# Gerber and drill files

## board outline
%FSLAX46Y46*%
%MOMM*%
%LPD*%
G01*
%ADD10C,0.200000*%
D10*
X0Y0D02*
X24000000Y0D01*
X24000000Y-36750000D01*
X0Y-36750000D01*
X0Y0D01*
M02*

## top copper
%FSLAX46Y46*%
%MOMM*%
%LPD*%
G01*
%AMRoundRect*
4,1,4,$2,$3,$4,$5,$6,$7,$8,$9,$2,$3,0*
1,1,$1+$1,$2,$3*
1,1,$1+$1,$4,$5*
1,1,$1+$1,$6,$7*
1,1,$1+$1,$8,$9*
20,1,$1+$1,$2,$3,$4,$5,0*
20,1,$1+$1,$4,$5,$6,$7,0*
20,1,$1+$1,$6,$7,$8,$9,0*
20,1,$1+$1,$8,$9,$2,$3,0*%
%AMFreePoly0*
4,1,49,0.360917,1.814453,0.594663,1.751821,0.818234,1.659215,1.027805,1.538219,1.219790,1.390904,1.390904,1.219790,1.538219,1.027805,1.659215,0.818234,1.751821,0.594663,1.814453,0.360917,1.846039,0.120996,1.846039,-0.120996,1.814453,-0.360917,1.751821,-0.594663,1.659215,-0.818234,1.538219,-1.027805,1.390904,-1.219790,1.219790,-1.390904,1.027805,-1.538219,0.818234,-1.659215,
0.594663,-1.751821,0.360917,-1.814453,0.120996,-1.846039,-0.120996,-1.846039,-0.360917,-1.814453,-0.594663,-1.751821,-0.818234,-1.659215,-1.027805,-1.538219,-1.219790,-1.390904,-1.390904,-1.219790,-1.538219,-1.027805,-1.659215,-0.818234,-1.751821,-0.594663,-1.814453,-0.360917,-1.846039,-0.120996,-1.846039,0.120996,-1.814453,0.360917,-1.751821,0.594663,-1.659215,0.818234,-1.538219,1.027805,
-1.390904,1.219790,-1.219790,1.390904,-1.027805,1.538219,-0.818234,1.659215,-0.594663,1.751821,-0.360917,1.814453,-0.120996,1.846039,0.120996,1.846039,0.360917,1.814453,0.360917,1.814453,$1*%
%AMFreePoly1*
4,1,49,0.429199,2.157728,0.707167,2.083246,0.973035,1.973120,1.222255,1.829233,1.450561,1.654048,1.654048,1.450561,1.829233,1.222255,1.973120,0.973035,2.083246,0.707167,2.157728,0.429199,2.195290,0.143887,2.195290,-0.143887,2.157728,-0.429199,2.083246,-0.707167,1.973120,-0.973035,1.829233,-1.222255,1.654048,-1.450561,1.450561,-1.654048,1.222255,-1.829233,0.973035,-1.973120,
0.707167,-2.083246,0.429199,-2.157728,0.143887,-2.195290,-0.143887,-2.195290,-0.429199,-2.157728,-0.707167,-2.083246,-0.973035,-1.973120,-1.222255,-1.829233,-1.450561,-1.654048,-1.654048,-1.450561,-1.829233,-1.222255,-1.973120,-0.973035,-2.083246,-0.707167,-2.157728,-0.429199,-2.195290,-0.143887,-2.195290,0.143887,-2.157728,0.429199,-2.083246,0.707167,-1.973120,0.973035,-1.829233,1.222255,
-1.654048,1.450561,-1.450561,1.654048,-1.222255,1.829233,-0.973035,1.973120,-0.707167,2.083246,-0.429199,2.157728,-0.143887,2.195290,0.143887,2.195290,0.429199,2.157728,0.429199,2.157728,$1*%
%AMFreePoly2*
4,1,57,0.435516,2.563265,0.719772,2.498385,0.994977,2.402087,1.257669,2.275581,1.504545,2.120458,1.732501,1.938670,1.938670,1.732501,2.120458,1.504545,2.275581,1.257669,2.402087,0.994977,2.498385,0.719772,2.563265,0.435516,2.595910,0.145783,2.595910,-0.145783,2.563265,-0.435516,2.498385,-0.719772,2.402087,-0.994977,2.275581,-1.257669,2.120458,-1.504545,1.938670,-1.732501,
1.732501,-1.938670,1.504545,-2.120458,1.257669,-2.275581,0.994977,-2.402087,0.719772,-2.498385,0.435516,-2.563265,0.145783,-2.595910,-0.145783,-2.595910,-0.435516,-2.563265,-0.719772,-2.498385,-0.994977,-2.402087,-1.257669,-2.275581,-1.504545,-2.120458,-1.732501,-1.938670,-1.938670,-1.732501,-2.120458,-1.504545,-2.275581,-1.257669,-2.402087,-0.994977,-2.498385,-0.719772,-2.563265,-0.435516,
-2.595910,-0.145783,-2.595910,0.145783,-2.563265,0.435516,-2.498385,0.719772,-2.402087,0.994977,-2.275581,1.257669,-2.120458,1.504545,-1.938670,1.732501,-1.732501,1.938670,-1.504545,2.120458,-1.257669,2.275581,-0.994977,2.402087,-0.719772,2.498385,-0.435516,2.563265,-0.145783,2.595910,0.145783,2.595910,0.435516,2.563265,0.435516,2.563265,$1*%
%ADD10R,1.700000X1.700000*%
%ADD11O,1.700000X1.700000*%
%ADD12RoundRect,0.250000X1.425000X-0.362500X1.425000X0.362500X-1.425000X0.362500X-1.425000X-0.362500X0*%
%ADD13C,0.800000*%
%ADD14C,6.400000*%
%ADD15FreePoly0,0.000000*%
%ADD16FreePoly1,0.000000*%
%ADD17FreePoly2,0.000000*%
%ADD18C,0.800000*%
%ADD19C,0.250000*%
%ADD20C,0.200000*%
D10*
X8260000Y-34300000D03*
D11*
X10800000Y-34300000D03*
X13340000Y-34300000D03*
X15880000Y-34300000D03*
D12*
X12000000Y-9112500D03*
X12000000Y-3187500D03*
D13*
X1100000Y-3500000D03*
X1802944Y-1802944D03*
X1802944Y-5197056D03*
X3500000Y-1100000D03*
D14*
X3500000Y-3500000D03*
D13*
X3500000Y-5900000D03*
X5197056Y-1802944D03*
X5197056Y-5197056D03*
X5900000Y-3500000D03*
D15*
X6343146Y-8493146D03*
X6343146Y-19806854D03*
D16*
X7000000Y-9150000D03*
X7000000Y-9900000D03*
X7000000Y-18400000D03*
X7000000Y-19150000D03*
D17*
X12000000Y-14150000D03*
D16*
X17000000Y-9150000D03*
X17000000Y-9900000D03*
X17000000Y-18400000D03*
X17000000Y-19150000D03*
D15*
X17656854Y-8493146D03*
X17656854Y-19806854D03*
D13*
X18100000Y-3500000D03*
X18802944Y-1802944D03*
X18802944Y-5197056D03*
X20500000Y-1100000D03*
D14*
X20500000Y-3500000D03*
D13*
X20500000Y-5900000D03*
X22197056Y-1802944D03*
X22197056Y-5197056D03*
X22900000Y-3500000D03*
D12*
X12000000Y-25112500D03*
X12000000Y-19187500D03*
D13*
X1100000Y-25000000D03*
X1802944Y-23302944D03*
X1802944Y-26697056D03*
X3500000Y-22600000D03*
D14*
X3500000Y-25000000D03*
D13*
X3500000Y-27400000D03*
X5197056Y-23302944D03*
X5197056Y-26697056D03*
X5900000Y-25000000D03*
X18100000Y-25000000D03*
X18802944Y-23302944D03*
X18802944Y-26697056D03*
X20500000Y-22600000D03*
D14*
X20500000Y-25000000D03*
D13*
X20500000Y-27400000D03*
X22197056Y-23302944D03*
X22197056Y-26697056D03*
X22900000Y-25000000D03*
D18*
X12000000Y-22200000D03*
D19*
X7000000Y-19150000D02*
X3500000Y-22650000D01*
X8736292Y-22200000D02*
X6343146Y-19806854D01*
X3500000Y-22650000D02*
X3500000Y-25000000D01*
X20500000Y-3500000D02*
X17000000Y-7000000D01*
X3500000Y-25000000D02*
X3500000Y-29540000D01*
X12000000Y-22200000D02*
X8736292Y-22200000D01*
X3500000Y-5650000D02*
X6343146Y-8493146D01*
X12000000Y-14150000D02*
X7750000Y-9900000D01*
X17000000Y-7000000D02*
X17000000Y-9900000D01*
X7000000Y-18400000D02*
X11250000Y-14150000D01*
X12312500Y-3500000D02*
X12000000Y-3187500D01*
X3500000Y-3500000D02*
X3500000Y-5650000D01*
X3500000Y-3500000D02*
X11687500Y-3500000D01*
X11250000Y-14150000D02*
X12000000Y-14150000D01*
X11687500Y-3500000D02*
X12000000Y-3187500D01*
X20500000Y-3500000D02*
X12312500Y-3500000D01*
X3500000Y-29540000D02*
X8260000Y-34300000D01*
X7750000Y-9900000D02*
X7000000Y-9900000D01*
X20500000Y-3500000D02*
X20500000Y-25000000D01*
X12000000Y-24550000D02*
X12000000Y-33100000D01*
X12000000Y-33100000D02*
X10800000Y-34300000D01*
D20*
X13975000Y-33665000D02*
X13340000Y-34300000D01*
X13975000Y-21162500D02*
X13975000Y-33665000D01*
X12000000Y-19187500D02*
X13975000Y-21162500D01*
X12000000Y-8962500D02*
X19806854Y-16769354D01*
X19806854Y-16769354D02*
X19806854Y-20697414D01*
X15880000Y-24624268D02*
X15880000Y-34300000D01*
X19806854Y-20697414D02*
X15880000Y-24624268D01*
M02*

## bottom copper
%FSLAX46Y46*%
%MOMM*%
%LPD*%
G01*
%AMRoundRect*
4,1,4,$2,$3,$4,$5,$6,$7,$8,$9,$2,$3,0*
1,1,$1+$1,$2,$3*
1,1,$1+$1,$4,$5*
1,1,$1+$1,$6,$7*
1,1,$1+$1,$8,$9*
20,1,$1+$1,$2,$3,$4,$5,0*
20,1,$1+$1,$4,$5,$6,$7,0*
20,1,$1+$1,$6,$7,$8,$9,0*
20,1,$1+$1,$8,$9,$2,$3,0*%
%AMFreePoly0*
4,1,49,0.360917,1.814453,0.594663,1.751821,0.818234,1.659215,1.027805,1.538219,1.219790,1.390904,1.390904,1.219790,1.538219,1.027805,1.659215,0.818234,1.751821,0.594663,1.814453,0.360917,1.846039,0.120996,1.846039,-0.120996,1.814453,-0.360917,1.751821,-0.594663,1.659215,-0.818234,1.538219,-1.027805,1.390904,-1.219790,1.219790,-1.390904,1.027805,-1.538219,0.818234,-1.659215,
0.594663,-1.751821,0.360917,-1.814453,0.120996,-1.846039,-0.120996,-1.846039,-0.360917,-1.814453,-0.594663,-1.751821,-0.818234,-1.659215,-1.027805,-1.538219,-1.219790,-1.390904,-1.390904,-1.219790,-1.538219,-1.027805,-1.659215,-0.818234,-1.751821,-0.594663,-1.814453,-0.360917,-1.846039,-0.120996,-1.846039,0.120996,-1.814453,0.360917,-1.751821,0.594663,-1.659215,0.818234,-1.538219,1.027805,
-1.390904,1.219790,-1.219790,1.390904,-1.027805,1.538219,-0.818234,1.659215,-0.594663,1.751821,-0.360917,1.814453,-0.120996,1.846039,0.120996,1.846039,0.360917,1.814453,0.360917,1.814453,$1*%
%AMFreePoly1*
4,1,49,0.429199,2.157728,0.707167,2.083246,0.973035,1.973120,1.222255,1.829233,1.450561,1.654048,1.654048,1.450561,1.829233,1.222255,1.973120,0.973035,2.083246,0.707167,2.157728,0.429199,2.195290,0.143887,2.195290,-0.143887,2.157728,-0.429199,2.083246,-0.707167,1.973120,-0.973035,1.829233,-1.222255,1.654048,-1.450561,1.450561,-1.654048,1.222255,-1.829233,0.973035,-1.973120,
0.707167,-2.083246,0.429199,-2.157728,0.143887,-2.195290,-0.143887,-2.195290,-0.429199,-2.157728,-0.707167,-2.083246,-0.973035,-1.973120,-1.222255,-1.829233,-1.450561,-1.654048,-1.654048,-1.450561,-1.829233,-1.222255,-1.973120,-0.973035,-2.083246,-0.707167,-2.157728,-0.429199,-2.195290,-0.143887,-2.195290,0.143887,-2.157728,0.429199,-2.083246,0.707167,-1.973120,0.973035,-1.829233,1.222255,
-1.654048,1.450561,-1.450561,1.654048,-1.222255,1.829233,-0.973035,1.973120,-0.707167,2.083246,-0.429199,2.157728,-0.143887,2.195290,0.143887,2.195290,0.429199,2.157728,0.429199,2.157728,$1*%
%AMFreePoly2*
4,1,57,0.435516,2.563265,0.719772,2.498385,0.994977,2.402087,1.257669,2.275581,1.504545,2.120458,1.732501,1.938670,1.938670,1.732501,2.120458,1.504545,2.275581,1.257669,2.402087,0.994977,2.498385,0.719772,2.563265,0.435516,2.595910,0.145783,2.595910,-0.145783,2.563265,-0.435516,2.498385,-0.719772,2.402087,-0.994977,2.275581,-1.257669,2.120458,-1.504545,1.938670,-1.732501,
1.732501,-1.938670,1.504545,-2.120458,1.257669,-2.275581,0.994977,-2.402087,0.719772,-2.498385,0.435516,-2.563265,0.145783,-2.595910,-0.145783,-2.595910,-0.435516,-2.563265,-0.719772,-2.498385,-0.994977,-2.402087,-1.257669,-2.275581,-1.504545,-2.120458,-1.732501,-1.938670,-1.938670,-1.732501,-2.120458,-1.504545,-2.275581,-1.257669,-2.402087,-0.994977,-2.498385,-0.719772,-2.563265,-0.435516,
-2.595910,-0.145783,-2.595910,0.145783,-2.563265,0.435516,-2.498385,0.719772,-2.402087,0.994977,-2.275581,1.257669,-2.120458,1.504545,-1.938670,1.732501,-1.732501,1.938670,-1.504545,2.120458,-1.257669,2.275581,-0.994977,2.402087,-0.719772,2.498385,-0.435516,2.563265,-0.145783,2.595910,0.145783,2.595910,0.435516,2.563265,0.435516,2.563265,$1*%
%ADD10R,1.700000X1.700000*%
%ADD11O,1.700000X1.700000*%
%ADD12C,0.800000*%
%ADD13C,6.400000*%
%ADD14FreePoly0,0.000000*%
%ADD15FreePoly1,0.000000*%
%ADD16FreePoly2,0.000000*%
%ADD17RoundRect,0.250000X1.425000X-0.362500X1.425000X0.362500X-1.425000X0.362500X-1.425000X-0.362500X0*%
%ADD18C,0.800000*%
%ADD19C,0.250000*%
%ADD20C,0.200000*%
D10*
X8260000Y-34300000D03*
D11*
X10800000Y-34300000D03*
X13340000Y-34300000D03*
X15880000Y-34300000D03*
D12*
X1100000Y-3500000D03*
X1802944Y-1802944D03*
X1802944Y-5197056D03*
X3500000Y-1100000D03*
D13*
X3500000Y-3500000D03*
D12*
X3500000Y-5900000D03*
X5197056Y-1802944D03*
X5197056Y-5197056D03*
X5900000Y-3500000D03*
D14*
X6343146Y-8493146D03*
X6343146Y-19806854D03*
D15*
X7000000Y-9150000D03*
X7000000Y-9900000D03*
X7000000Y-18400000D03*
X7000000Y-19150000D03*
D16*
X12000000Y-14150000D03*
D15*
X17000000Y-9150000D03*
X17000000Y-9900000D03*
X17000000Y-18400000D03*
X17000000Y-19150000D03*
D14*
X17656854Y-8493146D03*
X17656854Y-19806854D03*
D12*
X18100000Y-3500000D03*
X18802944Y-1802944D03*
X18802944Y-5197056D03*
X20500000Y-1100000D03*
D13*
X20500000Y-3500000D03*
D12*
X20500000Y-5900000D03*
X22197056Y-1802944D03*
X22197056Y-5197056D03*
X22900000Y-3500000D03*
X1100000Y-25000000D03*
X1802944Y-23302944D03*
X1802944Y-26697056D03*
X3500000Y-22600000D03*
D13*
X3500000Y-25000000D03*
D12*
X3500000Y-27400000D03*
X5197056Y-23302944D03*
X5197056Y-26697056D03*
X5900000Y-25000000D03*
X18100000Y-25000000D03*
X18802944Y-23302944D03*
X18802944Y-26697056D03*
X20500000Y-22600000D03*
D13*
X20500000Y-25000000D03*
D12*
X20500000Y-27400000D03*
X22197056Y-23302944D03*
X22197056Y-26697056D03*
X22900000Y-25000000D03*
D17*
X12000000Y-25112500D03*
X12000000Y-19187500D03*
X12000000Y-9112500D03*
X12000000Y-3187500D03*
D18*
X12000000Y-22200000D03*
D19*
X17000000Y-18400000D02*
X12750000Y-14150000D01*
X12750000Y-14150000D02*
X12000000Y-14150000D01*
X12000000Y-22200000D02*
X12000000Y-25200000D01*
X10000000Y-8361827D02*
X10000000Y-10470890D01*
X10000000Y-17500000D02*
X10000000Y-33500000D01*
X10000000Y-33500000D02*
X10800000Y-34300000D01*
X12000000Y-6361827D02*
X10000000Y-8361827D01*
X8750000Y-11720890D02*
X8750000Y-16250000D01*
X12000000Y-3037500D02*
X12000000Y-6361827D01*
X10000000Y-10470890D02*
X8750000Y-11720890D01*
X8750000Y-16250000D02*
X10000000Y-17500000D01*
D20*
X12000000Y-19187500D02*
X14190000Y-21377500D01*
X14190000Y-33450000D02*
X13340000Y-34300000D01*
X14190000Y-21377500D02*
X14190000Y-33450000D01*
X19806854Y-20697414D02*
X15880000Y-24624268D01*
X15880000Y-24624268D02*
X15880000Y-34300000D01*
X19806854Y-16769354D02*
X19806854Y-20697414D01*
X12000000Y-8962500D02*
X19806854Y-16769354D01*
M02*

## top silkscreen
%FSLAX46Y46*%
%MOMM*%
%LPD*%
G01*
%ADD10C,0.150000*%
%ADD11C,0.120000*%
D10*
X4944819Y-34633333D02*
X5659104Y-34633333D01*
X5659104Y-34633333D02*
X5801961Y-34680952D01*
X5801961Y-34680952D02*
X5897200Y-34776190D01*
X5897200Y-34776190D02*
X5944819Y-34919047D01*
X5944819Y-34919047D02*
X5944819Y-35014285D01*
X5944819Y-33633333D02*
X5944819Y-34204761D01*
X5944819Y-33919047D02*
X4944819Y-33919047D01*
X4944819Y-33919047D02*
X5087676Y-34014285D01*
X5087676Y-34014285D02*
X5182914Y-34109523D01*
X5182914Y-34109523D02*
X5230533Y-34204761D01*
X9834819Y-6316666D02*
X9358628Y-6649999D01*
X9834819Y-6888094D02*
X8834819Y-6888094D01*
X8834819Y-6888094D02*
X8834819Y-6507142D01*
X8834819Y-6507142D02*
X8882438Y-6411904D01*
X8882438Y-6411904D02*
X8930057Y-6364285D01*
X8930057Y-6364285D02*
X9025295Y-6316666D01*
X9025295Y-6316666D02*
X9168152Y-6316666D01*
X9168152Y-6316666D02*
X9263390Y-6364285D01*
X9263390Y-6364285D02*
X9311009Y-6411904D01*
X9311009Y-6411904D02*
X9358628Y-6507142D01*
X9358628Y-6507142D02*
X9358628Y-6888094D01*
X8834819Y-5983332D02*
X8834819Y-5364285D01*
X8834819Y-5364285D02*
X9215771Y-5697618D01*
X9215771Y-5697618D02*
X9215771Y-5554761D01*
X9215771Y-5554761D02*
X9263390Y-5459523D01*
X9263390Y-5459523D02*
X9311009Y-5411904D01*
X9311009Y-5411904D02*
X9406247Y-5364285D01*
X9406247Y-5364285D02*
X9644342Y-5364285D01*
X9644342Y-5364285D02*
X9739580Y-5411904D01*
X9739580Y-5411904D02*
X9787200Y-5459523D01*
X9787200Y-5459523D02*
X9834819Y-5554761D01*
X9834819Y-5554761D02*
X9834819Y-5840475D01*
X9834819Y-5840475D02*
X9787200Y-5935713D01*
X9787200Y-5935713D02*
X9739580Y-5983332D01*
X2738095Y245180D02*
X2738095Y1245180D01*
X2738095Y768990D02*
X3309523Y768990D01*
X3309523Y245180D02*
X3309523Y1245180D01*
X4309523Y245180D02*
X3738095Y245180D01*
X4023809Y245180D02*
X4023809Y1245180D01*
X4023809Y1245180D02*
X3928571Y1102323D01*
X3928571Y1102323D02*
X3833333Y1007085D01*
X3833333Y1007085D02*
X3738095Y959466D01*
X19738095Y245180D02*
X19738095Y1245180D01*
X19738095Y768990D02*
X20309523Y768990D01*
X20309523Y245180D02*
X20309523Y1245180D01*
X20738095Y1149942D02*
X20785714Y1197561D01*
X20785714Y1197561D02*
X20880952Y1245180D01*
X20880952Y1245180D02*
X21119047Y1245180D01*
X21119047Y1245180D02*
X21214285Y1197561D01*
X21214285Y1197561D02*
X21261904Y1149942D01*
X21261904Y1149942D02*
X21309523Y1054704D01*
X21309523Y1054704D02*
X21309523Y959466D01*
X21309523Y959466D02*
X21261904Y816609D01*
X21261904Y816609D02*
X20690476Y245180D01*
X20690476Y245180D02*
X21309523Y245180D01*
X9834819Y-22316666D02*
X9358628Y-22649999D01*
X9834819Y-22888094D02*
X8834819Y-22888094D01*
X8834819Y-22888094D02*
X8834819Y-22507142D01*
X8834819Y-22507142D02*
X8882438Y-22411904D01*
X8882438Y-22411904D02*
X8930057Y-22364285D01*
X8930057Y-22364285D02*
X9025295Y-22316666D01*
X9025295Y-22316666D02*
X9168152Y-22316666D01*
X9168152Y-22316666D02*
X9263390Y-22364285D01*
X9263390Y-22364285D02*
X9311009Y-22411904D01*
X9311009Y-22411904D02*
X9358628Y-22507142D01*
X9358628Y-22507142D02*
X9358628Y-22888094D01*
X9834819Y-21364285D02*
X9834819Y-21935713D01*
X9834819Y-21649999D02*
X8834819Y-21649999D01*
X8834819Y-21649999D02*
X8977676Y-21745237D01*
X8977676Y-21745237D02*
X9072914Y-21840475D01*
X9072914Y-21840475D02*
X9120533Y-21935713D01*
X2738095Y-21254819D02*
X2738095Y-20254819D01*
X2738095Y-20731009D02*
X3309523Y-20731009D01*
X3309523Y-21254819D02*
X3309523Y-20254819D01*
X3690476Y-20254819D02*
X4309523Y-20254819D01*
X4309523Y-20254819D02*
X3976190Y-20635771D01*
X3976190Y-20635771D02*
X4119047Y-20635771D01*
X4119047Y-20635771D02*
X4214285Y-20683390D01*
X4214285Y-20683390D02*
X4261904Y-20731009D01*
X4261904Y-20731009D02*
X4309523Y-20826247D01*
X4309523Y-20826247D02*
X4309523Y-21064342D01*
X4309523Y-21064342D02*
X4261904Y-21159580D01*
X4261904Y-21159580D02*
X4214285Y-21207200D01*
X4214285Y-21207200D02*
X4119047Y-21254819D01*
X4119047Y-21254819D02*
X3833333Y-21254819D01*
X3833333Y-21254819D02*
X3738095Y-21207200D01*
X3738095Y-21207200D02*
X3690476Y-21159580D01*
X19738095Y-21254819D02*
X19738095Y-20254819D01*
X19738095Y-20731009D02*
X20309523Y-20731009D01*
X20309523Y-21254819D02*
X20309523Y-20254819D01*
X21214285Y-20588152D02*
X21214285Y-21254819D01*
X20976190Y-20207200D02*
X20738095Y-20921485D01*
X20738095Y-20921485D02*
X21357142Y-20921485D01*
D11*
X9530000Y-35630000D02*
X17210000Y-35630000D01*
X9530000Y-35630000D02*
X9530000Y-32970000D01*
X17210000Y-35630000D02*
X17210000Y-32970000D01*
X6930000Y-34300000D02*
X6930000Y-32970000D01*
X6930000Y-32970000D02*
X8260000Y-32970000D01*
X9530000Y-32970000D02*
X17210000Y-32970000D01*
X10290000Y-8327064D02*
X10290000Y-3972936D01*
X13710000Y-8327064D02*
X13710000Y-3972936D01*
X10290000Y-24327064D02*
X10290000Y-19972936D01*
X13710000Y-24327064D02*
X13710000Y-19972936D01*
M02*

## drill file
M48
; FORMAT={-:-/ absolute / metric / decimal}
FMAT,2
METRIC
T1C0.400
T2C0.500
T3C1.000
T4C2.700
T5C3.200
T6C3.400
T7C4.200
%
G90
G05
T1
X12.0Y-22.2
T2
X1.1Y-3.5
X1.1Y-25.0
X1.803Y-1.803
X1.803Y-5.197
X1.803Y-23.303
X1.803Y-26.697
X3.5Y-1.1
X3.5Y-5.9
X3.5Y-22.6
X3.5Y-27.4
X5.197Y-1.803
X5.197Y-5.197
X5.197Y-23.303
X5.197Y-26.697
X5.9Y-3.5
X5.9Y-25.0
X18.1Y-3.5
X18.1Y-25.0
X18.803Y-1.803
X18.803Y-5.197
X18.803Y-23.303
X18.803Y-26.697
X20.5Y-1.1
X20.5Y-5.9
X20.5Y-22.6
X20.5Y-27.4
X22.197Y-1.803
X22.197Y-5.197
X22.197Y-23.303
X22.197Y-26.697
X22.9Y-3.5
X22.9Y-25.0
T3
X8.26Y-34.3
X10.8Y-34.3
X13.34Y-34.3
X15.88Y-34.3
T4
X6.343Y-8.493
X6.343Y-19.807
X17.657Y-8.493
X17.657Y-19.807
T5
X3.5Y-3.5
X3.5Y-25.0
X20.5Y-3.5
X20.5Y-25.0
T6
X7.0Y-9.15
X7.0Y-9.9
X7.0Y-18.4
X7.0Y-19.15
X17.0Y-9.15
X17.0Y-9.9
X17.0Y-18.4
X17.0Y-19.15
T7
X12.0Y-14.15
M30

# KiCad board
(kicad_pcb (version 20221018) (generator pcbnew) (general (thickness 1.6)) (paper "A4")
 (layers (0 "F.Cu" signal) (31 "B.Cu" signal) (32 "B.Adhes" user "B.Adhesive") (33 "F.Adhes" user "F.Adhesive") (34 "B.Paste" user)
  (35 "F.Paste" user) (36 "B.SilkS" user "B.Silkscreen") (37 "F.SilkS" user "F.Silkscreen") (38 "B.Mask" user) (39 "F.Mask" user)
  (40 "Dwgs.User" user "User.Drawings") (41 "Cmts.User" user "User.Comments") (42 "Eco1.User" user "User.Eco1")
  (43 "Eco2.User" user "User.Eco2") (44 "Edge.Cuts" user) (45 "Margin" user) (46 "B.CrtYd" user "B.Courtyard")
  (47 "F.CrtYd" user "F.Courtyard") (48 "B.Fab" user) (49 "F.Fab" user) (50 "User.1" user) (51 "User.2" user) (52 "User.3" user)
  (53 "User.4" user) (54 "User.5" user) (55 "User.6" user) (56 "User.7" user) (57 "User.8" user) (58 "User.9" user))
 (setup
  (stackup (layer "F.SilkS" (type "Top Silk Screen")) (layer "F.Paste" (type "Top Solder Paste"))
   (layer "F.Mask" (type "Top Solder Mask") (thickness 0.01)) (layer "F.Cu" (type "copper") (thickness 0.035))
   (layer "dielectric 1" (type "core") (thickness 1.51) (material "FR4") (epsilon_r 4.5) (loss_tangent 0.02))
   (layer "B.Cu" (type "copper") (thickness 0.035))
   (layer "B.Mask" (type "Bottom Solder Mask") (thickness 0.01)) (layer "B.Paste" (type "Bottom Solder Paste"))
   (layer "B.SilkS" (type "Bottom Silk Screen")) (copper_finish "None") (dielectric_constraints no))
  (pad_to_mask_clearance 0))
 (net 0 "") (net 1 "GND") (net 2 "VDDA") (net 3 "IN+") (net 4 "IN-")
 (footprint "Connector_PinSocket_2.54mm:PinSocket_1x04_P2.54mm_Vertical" (layer "F.Cu") (at 8.26 34.3 90)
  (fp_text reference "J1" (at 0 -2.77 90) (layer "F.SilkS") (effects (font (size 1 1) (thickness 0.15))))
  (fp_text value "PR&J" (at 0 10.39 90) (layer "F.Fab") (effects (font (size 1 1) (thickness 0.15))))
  (fp_line (start -1.33 1.27) (end -1.33 8.95) (stroke (width 0.12) (type solid)) (layer "F.SilkS"))
  (fp_line (start -1.33 1.27) (end 1.33 1.27) (stroke (width 0.12) (type solid)) (layer "F.SilkS"))
  (fp_line (start -1.33 8.95) (end 1.33 8.95) (stroke (width 0.12) (type solid)) (layer "F.SilkS"))
  (fp_line (start 0 -1.33) (end 1.33 -1.33) (stroke (width 0.12) (type solid)) (layer "F.SilkS"))
  (fp_line (start 1.33 -1.33) (end 1.33 0) (stroke (width 0.12) (type solid)) (layer "F.SilkS"))
  (fp_line (start 1.33 1.27) (end 1.33 8.95) (stroke (width 0.12) (type solid)) (layer "F.SilkS"))
  (pad "1" thru_hole rect (at 0 0 90) (size 1.7 1.7) (drill 1) (layers "*.Cu" "*.Mask") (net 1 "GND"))
  (pad "2" thru_hole oval (at 0 2.54 90) (size 1.7 1.7) (drill 1) (layers "*.Cu" "*.Mask") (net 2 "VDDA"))
  (pad "3" thru_hole oval (at 0 5.08 90) (size 1.7 1.7) (drill 1) (layers "*.Cu" "*.Mask") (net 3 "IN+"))
  (pad "4" thru_hole oval (at 0 7.62 90) (size 1.7 1.7) (drill 1) (layers "*.Cu" "*.Mask") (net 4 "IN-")))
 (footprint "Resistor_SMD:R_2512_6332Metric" (layer "F.Cu") (at 12 6.15 90)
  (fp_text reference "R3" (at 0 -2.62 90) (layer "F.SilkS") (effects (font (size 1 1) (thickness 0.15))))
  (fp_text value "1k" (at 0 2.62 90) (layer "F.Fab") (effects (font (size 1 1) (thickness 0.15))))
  (fp_line (start -2.177064 -1.71) (end 2.177064 -1.71) (stroke (width 0.12) (type solid)) (layer "F.SilkS"))
  (fp_line (start -2.177064 1.71) (end 2.177064 1.71) (stroke (width 0.12) (type solid)) (layer "F.SilkS"))
  (pad "1" smd roundrect (at -2.9625 0 90) (size 1.225 3.35) (layers "F.Cu" "F.Paste" "F.Mask") (roundrect_rratio 0.2040816327)
   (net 4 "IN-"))
  (pad "2" smd roundrect (at 2.9625 0 90) (size 1.225 3.35) (layers "F.Cu" "F.Paste" "F.Mask") (roundrect_rratio 0.2040816327) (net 1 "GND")))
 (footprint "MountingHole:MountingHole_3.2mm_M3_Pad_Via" (layer "F.Cu") (at 3.5 3.5)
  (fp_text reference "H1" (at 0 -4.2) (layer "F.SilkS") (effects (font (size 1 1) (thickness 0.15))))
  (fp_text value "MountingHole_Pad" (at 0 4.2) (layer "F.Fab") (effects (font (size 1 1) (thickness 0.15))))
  (pad "1" thru_hole circle (at -2.4 0) (size 0.8 0.8) (drill 0.5) (layers "*.Cu" "*.Mask") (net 1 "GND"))
  (pad "1" thru_hole circle (at -1.697056 -1.697056) (size 0.8 0.8) (drill 0.5) (layers "*.Cu" "*.Mask") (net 1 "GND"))
  (pad "1" thru_hole circle (at -1.697056 1.697056) (size 0.8 0.8) (drill 0.5) (layers "*.Cu" "*.Mask") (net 1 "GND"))
  (pad "1" thru_hole circle (at 0 -2.4) (size 0.8 0.8) (drill 0.5) (layers "*.Cu" "*.Mask") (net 1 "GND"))
  (pad "1" thru_hole circle (at 0 0) (size 6.4 6.4) (drill 3.2) (layers "*.Cu" "*.Mask") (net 1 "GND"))
  (pad "1" thru_hole circle (at 0 2.4) (size 0.8 0.8) (drill 0.5) (layers "*.Cu" "*.Mask") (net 1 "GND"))
  (pad "1" thru_hole circle (at 1.697056 -1.697056) (size 0.8 0.8) (drill 0.5) (layers "*.Cu" "*.Mask") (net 1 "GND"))
  (pad "1" thru_hole circle (at 1.697056 1.697056) (size 0.8 0.8) (drill 0.5) (layers "*.Cu" "*.Mask") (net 1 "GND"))
  (pad "1" thru_hole circle (at 2.4 0) (size 0.8 0.8) (drill 0.5) (layers "*.Cu" "*.Mask") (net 1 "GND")))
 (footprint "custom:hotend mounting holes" (layer "F.Cu") (at 12 14.15)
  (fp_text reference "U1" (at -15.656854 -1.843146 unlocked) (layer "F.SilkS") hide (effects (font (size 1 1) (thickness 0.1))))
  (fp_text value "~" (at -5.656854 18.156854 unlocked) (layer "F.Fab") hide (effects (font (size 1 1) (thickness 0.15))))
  (pad "1" thru_hole custom (at -5.656854 -5.656854) (size 3.7 3.7) (drill 2.7) (layers "*.Cu" "*.Mask") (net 1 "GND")
   (thermal_bridge_angle 45) (options (clearance outline) (anchor circle)) (primitives))
  (pad "1" thru_hole custom (at -5.656854 5.656854) (size 3.7 3.7) (drill 2.7) (layers "*.Cu" "*.Mask") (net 1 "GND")
   (thermal_bridge_angle 45) (options (clearance outline) (anchor circle)) (primitives))
  (pad "1" thru_hole custom (at -5 -5) (size 4.4 4.4) (drill 3.4) (layers "*.Cu" "*.Mask") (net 1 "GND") (thermal_bridge_angle 45)
   (options (clearance outline) (anchor circle)) (primitives))
  (pad "1" thru_hole custom (at -5 -4.25) (size 4.4 4.4) (drill 3.4) (layers "*.Cu" "*.Mask") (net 1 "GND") (thermal_bridge_angle 45)
   (options (clearance outline) (anchor circle)) (primitives))
  (pad "1" thru_hole custom (at -5 4.25) (size 4.4 4.4) (drill 3.4) (layers "*.Cu" "*.Mask") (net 1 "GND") (thermal_bridge_angle 45)
   (options (clearance outline) (anchor circle)) (primitives))
  (pad "1" thru_hole custom (at -5 5) (size 4.4 4.4) (drill 3.4) (layers "*.Cu" "*.Mask") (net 1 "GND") (thermal_bridge_angle 45)
   (options (clearance outline) (anchor circle)) (primitives))
  (pad "1" thru_hole custom (at 0 0) (size 5.2 5.2) (drill 4.2) (layers "*.Cu" "*.Mask") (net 1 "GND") (thermal_bridge_angle 45)
   (options (clearance outline) (anchor circle)) (primitives))
  (pad "1" thru_hole custom (at 5 -5) (size 4.4 4.4) (drill 3.4) (layers "*.Cu" "*.Mask") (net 1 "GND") (thermal_bridge_angle 45)
   (options (clearance outline) (anchor circle)) (primitives))
  (pad "1" thru_hole custom (at 5 -4.25) (size 4.4 4.4) (drill 3.4) (layers "*.Cu" "*.Mask") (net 1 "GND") (thermal_bridge_angle 45)
   (options (clearance outline) (anchor circle)) (primitives))
  (pad "1" thru_hole custom (at 5 4.25) (size 4.4 4.4) (drill 3.4) (layers "*.Cu" "*.Mask") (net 1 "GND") (thermal_bridge_angle 45)
   (options (clearance outline) (anchor circle)) (primitives))
  (pad "1" thru_hole custom (at 5 5) (size 4.4 4.4) (drill 3.4) (layers "*.Cu" "*.Mask") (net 1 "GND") (thermal_bridge_angle 45)
   (options (clearance outline) (anchor circle)) (primitives))
  (pad "1" thru_hole custom (at 5.656854 -5.656854) (size 3.7 3.7) (drill 2.7) (layers "*.Cu" "*.Mask") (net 1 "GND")
   (thermal_bridge_angle 45) (options (clearance outline) (anchor circle)) (primitives))
  (pad "1" thru_hole custom (at 5.656854 5.656854) (size 3.7 3.7) (drill 2.7) (layers "*.Cu" "*.Mask") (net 1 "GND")
   (thermal_bridge_angle 45) (options (clearance outline) (anchor circle)) (primitives)))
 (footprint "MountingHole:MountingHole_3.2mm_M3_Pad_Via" (layer "F.Cu") (at 20.5 3.5)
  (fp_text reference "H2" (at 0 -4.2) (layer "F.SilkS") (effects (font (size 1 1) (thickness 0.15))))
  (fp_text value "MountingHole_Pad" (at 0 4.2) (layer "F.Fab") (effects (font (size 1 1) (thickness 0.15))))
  (pad "1" thru_hole circle (at -2.4 0) (size 0.8 0.8) (drill 0.5) (layers "*.Cu" "*.Mask") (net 1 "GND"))
  (pad "1" thru_hole circle (at -1.697056 -1.697056) (size 0.8 0.8) (drill 0.5) (layers "*.Cu" "*.Mask") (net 1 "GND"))
  (pad "1" thru_hole circle (at -1.697056 1.697056) (size 0.8 0.8) (drill 0.5) (layers "*.Cu" "*.Mask") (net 1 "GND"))
  (pad "1" thru_hole circle (at 0 -2.4) (size 0.8 0.8) (drill 0.5) (layers "*.Cu" "*.Mask") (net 1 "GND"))
  (pad "1" thru_hole circle (at 0 0) (size 6.4 6.4) (drill 3.2) (layers "*.Cu" "*.Mask") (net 1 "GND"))
  (pad "1" thru_hole circle (at 0 2.4) (size 0.8 0.8) (drill 0.5) (layers "*.Cu" "*.Mask") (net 1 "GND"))
  (pad "1" thru_hole circle (at 1.697056 -1.697056) (size 0.8 0.8) (drill 0.5) (layers "*.Cu" "*.Mask") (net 1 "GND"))
  (pad "1" thru_hole circle (at 1.697056 1.697056) (size 0.8 0.8) (drill 0.5) (layers "*.Cu" "*.Mask") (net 1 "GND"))
  (pad "1" thru_hole circle (at 2.4 0) (size 0.8 0.8) (drill 0.5) (layers "*.Cu" "*.Mask") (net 1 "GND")))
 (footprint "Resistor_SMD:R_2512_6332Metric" (layer "F.Cu") (at 12 22.15 90)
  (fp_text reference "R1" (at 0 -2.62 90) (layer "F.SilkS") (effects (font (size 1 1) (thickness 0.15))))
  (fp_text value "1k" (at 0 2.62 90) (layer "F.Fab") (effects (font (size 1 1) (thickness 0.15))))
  (fp_line (start -2.177064 -1.71) (end 2.177064 -1.71) (stroke (width 0.12) (type solid)) (layer "F.SilkS"))
  (fp_line (start -2.177064 1.71) (end 2.177064 1.71) (stroke (width 0.12) (type solid)) (layer "F.SilkS"))
  (pad "1" smd roundrect (at -2.9625 0 90) (size 1.225 3.35) (layers "F.Cu" "F.Paste" "F.Mask") (roundrect_rratio 0.2040816327)
   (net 2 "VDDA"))
  (pad "2" smd roundrect (at 2.9625 0 90) (size 1.225 3.35) (layers "F.Cu" "F.Paste" "F.Mask") (roundrect_rratio 0.2040816327) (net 3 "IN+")))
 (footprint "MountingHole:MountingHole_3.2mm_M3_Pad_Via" (layer "F.Cu") (at 3.5 25)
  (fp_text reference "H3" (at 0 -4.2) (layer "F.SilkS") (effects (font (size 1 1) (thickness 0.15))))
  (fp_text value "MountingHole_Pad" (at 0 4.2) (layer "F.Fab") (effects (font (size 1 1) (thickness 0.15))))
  (pad "1" thru_hole circle (at -2.4 0) (size 0.8 0.8) (drill 0.5) (layers "*.Cu" "*.Mask") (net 1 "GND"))
  (pad "1" thru_hole circle (at -1.697056 -1.697056) (size 0.8 0.8) (drill 0.5) (layers "*.Cu" "*.Mask") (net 1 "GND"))
  (pad "1" thru_hole circle (at -1.697056 1.697056) (size 0.8 0.8) (drill 0.5) (layers "*.Cu" "*.Mask") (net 1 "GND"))
  (pad "1" thru_hole circle (at 0 -2.4) (size 0.8 0.8) (drill 0.5) (layers "*.Cu" "*.Mask") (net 1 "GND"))
  (pad "1" thru_hole circle (at 0 0) (size 6.4 6.4) (drill 3.2) (layers "*.Cu" "*.Mask") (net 1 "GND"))
  (pad "1" thru_hole circle (at 0 2.4) (size 0.8 0.8) (drill 0.5) (layers "*.Cu" "*.Mask") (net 1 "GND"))
  (pad "1" thru_hole circle (at 1.697056 -1.697056) (size 0.8 0.8) (drill 0.5) (layers "*.Cu" "*.Mask") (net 1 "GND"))
  (pad "1" thru_hole circle (at 1.697056 1.697056) (size 0.8 0.8) (drill 0.5) (layers "*.Cu" "*.Mask") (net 1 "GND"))
  (pad "1" thru_hole circle (at 2.4 0) (size 0.8 0.8) (drill 0.5) (layers "*.Cu" "*.Mask") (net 1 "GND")))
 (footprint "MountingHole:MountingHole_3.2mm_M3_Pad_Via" (layer "F.Cu") (at 20.5 25)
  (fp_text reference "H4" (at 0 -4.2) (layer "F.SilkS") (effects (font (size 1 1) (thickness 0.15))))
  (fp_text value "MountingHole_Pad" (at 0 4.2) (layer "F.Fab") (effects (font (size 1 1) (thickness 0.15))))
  (pad "1" thru_hole circle (at -2.4 0) (size 0.8 0.8) (drill 0.5) (layers "*.Cu" "*.Mask") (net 1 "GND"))
  (pad "1" thru_hole circle (at -1.697056 -1.697056) (size 0.8 0.8) (drill 0.5) (layers "*.Cu" "*.Mask") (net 1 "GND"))
  (pad "1" thru_hole circle (at -1.697056 1.697056) (size 0.8 0.8) (drill 0.5) (layers "*.Cu" "*.Mask") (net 1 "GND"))
  (pad "1" thru_hole circle (at 0 -2.4) (size 0.8 0.8) (drill 0.5) (layers "*.Cu" "*.Mask") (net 1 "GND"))
  (pad "1" thru_hole circle (at 0 0) (size 6.4 6.4) (drill 3.2) (layers "*.Cu" "*.Mask") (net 1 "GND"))
  (pad "1" thru_hole circle (at 0 2.4) (size 0.8 0.8) (drill 0.5) (layers "*.Cu" "*.Mask") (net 1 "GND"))
  (pad "1" thru_hole circle (at 1.697056 -1.697056) (size 0.8 0.8) (drill 0.5) (layers "*.Cu" "*.Mask") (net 1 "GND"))
  (pad "1" thru_hole circle (at 1.697056 1.697056) (size 0.8 0.8) (drill 0.5) (layers "*.Cu" "*.Mask") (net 1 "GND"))
  (pad "1" thru_hole circle (at 2.4 0) (size 0.8 0.8) (drill 0.5) (layers "*.Cu" "*.Mask") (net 1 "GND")))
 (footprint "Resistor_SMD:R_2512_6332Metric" (layer "B.Cu") (at 12 22.15 90)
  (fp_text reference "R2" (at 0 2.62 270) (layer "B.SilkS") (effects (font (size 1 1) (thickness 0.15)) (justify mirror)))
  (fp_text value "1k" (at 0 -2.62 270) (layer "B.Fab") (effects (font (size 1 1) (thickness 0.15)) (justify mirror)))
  (pad "1" smd roundrect (at -2.9625 0 90) (size 1.225 3.35) (layers "B.Cu" "B.Paste" "B.Mask") (roundrect_rratio 0.2040816327)
   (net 1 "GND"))
  (pad "2" smd roundrect (at 2.9625 0 90) (size 1.225 3.35) (layers "B.Cu" "B.Paste" "B.Mask") (roundrect_rratio 0.2040816327) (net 3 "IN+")))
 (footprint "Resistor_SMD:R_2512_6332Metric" (layer "B.Cu") (at 12 6.15 90)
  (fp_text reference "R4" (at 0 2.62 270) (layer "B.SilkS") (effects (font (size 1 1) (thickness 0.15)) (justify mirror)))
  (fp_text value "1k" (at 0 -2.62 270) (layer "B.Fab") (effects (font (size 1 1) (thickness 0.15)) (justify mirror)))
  (pad "1" smd roundrect (at -2.9625 0 90) (size 1.225 3.35) (layers "B.Cu" "B.Paste" "B.Mask") (roundrect_rratio 0.2040816327)
   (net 4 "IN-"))
  (pad "2" smd roundrect (at 2.9625 0 90) (size 1.225 3.35) (layers "B.Cu" "B.Paste" "B.Mask") (roundrect_rratio 0.2040816327)
   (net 2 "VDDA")))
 (gr_rect (start 0 0) (end 24 36.75) (stroke (width 0.2) (type default)) (fill none) (layer "Edge.Cuts"))
 (segment (start 7 19.15) (end 3.5 22.65) (width 0.25) (layer "F.Cu") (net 1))
 (segment (start 8.736292 22.2) (end 6.343146 19.806854) (width 0.25) (layer "F.Cu") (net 1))
 (segment (start 3.5 22.65) (end 3.5 25) (width 0.25) (layer "F.Cu") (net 1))
 (segment (start 20.5 3.5) (end 17 7) (width 0.25) (layer "F.Cu") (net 1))
 (segment (start 3.5 25) (end 3.5 29.54) (width 0.25) (layer "F.Cu") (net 1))
 (segment (start 12 22.2) (end 8.736292 22.2) (width 0.25) (layer "F.Cu") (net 1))
 (segment (start 3.5 5.65) (end 6.343146 8.493146) (width 0.25) (layer "F.Cu") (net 1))
 (segment (start 12 14.15) (end 7.75 9.9) (width 0.25) (layer "F.Cu") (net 1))
 (segment (start 17 7) (end 17 9.9) (width 0.25) (layer "F.Cu") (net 1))
 (segment (start 7 18.4) (end 11.25 14.15) (width 0.25) (layer "F.Cu") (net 1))
 (segment (start 12.3125 3.5) (end 12 3.1875) (width 0.25) (layer "F.Cu") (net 1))
 (segment (start 3.5 3.5) (end 3.5 5.65) (width 0.25) (layer "F.Cu") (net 1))
 (segment (start 3.5 3.5) (end 11.6875 3.5) (width 0.25) (layer "F.Cu") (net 1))
 (segment (start 11.25 14.15) (end 12 14.15) (width 0.25) (layer "F.Cu") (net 1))
 (segment (start 11.6875 3.5) (end 12 3.1875) (width 0.25) (layer "F.Cu") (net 1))
 (segment (start 20.5 3.5) (end 12.3125 3.5) (width 0.25) (layer "F.Cu") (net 1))
 (segment (start 3.5 29.54) (end 8.26 34.3) (width 0.25) (layer "F.Cu") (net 1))
 (segment (start 7.75 9.9) (end 7 9.9) (width 0.25) (layer "F.Cu") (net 1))
 (segment (start 20.5 3.5) (end 20.5 25) (width 0.25) (layer "F.Cu") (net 1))
 (via (at 12 22.2) (size 0.8) (drill 0.4) (layers "F.Cu" "B.Cu") (free) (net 1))
 (segment (start 17 18.4) (end 12.75 14.15) (width 0.25) (layer "B.Cu") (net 1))
 (segment (start 12.75 14.15) (end 12 14.15) (width 0.25) (layer "B.Cu") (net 1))
 (segment (start 12 22.2) (end 12 25.2) (width 0.25) (layer "B.Cu") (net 1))
 (segment (start 12 24.55) (end 12 33.1) (width 0.25) (layer "F.Cu") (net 2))
 (segment (start 12 33.1) (end 10.8 34.3) (width 0.25) (layer "F.Cu") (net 2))
 (segment (start 10 8.361827) (end 10 10.47089) (width 0.25) (layer "B.Cu") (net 2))
 (segment (start 10 17.5) (end 10 33.5) (width 0.25) (layer "B.Cu") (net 2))
 (segment (start 10 33.5) (end 10.8 34.3) (width 0.25) (layer "B.Cu") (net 2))
 (segment (start 12 6.361827) (end 10 8.361827) (width 0.25) (layer "B.Cu") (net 2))
 (segment (start 8.75 11.72089) (end 8.75 16.25) (width 0.25) (layer "B.Cu") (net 2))
 (segment (start 12 3.0375) (end 12 6.361827) (width 0.25) (layer "B.Cu") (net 2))
 (segment (start 10 10.47089) (end 8.75 11.72089) (width 0.25) (layer "B.Cu") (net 2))
 (segment (start 8.75 16.25) (end 10 17.5) (width 0.25) (layer "B.Cu") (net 2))
 (segment (start 13.975 33.665) (end 13.34 34.3) (width 0.2) (layer "F.Cu") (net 3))
 (segment (start 13.975 21.1625) (end 13.975 33.665) (width 0.2) (layer "F.Cu") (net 3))
 (segment (start 12 19.1875) (end 13.975 21.1625) (width 0.2) (layer "F.Cu") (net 3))
 (segment (start 12 19.1875) (end 14.19 21.3775) (width 0.2) (layer "B.Cu") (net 3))
 (segment (start 14.19 33.45) (end 13.34 34.3) (width 0.2) (layer "B.Cu") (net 3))
 (segment (start 14.19 21.3775) (end 14.19 33.45) (width 0.2) (layer "B.Cu") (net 3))
 (segment (start 12 8.9625) (end 19.806854 16.769354) (width 0.2) (layer "F.Cu") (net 4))
 (segment (start 19.806854 16.769354) (end 19.806854 20.697414) (width 0.2) (layer "F.Cu") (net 4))
 (segment (start 15.88 24.624268) (end 15.88 34.3) (width 0.2) (layer "F.Cu") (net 4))
 (segment (start 19.806854 20.697414) (end 15.88 24.624268) (width 0.2) (layer "F.Cu") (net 4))
 (segment (start 19.806854 20.697414) (end 15.88 24.624268) (width 0.2) (layer "B.Cu") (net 4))
 (segment (start 15.88 24.624268) (end 15.88 34.3) (width 0.2) (layer "B.Cu") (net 4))
 (segment (start 19.806854 16.769354) (end 19.806854 20.697414) (width 0.2) (layer "B.Cu") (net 4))
 (segment (start 12 8.9625) (end 19.806854 16.769354) (width 0.2) (layer "B.Cu") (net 4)))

